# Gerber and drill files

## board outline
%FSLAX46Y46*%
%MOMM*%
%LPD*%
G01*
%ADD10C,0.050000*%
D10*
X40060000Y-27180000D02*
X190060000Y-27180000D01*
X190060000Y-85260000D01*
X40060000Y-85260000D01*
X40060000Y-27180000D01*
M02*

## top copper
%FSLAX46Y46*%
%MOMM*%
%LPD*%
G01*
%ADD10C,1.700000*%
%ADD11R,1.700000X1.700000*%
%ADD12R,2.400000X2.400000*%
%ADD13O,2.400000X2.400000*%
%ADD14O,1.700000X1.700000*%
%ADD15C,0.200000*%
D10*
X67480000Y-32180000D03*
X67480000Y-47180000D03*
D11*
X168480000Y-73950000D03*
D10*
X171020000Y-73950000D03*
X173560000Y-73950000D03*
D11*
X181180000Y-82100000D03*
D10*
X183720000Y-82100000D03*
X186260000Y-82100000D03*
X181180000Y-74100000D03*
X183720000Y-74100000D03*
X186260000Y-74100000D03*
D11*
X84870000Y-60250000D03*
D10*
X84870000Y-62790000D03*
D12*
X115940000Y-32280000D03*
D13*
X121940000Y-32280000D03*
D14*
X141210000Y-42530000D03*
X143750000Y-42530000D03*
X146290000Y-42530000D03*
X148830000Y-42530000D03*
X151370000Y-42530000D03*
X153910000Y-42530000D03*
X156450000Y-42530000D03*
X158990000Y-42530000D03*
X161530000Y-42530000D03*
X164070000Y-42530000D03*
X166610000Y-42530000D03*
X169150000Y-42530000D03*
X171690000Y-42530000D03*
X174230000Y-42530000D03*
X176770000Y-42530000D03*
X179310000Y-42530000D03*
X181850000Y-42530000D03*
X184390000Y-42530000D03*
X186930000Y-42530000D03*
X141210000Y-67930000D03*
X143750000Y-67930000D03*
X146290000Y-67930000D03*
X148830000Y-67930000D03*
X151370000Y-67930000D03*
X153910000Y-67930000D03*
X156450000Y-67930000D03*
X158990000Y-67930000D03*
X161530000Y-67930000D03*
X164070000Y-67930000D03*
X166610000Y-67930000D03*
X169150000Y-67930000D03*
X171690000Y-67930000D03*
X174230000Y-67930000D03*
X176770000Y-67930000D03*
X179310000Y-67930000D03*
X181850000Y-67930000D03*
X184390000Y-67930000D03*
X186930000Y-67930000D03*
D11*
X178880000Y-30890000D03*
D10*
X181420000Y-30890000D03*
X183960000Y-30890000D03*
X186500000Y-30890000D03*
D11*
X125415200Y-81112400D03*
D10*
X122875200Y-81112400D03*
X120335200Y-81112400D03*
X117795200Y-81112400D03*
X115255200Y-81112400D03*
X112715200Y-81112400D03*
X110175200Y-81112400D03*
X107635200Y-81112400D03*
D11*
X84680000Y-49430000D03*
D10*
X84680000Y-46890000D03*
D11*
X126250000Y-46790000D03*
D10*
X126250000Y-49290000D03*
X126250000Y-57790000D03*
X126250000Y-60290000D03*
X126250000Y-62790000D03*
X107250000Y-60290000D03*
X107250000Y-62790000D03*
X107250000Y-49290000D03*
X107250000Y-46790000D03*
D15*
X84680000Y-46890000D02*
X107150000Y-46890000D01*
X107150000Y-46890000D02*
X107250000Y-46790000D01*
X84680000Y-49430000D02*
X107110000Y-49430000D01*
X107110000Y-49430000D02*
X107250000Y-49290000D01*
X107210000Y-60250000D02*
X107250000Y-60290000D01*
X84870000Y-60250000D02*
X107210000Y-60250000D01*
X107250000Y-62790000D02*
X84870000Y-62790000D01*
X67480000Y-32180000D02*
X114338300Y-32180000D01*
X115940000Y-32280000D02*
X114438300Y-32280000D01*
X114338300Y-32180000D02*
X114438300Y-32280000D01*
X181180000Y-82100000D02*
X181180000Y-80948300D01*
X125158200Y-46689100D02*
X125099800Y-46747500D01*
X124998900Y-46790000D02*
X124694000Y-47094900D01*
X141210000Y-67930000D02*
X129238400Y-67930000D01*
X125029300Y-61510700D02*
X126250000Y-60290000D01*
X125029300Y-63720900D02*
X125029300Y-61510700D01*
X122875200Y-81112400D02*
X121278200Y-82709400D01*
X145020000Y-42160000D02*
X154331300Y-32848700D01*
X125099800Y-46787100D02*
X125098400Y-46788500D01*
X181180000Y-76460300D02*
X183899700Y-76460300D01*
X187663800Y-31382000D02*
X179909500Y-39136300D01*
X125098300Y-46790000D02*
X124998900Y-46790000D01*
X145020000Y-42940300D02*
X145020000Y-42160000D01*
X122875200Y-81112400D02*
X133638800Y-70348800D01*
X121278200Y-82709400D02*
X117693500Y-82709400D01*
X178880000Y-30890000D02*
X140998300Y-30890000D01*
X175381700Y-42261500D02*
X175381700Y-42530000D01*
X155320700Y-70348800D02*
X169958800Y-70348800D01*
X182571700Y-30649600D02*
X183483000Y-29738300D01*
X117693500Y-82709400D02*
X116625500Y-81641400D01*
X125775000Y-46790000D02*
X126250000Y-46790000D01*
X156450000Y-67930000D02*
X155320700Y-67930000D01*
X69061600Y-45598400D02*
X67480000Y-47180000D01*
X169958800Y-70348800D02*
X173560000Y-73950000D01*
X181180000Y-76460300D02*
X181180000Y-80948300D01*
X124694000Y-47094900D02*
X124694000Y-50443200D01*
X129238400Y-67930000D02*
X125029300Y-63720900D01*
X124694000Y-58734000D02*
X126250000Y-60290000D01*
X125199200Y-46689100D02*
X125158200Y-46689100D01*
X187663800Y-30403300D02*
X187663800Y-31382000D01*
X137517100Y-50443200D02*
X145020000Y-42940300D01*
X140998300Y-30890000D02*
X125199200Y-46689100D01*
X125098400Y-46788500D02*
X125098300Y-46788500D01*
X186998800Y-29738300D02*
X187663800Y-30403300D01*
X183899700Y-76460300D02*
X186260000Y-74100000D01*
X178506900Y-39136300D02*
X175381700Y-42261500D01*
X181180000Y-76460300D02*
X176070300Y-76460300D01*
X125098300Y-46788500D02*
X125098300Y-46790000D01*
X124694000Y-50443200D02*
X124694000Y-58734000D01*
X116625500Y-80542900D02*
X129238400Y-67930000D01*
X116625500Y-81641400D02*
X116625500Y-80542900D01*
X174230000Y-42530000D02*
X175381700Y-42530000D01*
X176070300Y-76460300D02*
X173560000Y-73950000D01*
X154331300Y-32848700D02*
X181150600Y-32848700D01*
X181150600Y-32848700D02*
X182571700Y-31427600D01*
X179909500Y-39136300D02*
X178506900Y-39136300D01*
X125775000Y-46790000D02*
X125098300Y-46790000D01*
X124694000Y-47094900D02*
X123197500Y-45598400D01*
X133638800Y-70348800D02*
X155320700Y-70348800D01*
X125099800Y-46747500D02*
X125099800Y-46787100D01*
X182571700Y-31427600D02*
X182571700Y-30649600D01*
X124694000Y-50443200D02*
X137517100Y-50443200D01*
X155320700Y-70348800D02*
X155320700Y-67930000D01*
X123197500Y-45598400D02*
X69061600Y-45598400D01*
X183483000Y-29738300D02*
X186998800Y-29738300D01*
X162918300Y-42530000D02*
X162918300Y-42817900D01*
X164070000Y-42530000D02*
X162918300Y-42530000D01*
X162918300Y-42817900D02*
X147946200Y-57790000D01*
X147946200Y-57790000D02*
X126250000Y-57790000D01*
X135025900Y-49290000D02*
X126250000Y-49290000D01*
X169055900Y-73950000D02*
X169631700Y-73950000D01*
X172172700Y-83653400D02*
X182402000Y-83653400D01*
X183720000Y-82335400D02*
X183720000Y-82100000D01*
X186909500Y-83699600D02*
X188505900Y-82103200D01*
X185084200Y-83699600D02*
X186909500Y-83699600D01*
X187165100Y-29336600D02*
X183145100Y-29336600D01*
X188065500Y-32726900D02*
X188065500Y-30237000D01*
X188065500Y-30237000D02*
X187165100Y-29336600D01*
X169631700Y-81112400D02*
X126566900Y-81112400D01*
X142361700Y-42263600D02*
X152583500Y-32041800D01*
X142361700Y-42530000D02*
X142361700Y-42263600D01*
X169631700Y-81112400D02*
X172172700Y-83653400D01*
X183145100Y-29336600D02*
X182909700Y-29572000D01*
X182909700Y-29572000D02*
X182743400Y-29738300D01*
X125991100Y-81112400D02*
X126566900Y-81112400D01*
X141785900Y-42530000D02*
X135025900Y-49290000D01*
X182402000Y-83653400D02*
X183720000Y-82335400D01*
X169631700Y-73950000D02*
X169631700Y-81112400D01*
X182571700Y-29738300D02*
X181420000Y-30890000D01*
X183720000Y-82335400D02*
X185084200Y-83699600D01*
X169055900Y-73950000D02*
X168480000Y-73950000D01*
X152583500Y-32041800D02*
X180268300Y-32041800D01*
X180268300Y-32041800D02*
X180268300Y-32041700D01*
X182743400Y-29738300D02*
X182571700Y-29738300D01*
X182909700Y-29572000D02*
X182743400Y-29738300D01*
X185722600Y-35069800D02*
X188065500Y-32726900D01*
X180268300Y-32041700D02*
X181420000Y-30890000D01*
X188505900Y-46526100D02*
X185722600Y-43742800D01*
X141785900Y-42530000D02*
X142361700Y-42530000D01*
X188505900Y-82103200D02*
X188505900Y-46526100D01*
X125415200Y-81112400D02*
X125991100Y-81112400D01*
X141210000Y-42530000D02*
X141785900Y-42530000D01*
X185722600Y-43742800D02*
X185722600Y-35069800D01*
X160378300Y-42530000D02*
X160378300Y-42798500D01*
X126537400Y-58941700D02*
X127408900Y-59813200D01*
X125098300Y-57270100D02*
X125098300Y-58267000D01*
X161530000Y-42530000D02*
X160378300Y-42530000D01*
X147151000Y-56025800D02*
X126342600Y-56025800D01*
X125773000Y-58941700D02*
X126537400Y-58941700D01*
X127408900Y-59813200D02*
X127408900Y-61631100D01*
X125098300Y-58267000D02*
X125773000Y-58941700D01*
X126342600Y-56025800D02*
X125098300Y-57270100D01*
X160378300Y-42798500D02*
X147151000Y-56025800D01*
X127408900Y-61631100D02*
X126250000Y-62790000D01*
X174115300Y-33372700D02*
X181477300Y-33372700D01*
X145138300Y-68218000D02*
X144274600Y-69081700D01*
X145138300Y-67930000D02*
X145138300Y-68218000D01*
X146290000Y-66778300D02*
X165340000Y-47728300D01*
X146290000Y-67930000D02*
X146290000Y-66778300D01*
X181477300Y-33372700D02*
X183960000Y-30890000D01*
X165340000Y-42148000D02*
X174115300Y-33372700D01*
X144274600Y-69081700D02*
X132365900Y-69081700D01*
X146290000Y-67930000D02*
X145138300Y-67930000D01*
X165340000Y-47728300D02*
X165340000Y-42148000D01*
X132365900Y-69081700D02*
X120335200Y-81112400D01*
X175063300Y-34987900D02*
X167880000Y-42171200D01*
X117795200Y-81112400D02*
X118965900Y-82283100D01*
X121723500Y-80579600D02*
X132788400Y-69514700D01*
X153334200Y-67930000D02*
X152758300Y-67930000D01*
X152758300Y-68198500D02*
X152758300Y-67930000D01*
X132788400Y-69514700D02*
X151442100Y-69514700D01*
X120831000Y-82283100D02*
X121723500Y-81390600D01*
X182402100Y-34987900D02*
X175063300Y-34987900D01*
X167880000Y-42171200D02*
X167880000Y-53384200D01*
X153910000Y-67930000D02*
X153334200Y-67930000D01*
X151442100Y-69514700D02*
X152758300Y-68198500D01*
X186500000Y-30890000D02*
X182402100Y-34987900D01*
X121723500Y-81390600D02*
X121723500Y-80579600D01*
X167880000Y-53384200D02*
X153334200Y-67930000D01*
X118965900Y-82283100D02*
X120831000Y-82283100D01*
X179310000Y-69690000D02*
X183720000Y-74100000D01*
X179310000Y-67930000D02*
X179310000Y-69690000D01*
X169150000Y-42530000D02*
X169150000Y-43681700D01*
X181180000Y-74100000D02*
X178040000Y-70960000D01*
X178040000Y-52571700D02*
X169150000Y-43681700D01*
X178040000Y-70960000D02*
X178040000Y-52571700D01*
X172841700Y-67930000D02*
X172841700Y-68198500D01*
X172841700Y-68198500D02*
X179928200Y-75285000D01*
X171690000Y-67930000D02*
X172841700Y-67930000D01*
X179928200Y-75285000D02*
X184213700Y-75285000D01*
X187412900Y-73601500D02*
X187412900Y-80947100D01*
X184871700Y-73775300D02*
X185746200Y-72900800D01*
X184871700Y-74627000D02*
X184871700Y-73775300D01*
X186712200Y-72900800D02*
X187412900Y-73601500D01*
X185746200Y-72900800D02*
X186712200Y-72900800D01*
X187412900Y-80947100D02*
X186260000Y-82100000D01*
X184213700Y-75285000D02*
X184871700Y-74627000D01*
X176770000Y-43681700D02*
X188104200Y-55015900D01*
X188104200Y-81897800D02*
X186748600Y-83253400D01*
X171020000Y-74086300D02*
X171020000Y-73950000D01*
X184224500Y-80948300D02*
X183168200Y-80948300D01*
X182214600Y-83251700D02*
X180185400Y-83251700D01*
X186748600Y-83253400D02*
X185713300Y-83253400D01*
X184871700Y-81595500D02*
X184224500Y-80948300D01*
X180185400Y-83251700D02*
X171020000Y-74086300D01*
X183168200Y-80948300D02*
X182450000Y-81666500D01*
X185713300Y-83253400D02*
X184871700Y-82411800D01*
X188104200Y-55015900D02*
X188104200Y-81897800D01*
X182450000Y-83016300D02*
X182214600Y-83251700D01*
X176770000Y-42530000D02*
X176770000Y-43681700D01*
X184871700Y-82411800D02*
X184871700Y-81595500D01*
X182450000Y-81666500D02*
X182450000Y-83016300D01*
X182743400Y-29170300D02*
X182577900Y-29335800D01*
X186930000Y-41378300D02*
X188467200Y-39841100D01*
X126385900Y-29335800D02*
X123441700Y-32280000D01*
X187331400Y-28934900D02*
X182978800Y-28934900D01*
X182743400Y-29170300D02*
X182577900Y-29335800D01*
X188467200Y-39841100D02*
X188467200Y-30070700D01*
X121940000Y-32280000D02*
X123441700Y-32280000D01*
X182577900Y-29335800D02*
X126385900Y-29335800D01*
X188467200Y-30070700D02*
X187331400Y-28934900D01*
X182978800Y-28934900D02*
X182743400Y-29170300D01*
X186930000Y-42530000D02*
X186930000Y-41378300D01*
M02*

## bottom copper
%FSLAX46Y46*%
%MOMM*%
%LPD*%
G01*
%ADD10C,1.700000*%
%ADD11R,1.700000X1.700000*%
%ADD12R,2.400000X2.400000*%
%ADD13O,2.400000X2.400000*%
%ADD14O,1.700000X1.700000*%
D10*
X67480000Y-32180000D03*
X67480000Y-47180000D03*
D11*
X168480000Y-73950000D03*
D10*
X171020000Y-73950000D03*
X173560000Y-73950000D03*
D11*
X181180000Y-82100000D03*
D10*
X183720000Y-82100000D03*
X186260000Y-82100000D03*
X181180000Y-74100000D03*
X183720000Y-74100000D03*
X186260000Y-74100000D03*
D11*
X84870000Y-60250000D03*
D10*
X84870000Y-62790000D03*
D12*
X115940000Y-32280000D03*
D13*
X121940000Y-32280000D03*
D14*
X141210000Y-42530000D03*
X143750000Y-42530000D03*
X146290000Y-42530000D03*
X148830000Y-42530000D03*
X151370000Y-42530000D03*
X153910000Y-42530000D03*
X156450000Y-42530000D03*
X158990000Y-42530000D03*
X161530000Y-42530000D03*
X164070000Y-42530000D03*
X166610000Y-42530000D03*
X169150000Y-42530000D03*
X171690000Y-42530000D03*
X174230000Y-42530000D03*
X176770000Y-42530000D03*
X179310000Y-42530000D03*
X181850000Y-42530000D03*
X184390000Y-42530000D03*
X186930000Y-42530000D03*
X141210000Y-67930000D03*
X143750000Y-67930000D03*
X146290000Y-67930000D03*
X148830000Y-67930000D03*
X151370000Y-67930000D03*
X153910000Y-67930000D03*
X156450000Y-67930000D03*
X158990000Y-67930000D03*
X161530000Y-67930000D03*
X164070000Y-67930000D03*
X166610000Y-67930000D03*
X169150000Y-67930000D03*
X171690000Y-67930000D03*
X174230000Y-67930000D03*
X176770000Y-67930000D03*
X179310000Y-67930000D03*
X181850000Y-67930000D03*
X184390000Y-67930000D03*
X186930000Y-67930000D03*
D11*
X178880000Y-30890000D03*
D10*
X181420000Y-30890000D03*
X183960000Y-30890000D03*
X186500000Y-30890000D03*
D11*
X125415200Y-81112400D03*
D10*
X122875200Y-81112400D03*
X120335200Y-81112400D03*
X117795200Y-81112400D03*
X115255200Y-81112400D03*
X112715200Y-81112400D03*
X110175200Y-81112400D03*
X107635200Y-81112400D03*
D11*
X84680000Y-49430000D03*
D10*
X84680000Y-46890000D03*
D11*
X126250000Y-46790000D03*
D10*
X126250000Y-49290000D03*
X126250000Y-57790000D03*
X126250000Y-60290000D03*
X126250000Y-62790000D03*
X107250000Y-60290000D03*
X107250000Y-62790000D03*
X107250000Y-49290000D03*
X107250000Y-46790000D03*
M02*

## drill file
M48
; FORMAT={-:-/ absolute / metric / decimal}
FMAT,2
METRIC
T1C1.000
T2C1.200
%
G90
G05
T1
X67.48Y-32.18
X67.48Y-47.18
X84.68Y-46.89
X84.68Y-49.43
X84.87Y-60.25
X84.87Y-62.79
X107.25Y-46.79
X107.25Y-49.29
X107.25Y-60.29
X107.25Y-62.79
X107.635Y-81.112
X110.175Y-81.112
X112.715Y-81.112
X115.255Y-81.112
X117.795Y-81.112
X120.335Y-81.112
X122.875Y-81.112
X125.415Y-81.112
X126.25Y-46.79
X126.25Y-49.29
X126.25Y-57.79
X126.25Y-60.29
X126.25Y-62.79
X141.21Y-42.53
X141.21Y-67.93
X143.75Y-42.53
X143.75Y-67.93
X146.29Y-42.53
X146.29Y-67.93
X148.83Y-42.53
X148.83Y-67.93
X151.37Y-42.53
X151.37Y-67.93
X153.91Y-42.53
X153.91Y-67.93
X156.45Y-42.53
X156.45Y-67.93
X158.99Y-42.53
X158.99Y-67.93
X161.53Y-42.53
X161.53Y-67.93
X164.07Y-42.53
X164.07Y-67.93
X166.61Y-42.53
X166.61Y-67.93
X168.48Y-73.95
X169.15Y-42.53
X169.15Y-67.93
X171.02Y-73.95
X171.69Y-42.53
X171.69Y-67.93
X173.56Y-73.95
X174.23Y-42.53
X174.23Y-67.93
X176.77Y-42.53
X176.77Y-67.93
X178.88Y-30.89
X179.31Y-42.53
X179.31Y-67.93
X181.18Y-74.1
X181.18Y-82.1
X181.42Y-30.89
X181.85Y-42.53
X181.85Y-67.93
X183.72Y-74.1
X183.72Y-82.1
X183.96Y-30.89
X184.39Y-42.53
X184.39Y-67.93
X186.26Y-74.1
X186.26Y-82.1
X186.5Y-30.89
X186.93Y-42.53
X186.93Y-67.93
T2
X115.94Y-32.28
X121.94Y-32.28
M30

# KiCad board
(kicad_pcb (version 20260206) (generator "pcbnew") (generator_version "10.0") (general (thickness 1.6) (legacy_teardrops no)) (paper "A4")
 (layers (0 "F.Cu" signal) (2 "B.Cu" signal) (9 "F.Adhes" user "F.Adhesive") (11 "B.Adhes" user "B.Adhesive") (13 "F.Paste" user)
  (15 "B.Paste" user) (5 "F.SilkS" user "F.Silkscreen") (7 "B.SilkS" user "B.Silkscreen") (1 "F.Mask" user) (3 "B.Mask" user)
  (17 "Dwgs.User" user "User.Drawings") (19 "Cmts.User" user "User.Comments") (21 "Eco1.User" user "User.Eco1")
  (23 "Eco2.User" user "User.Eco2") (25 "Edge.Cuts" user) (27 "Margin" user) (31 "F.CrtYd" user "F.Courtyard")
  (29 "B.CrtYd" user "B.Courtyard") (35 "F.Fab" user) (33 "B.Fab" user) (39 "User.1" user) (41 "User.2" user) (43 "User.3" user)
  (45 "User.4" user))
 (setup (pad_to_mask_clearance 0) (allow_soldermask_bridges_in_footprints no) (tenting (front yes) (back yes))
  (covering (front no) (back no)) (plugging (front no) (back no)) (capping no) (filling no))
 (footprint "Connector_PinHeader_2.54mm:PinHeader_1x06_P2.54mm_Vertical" (layer "F.Cu") (at 67.48 47.18 180)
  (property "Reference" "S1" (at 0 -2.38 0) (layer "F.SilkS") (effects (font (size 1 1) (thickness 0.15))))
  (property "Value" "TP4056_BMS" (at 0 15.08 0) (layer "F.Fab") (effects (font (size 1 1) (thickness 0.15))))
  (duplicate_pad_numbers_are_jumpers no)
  (pad "5" thru_hole circle (at 0 15 180) (size 1.7 1.7) (drill 1) (layers "*.Cu" "*.Mask") (remove_unused_layers no) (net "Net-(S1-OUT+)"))
  (pad "6" thru_hole circle (at 0 0 180) (size 1.7 1.7) (drill 1) (layers "*.Cu" "*.Mask") (remove_unused_layers no) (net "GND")))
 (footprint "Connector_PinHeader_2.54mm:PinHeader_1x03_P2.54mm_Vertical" (layer "F.Cu") (at 168.48 73.95 90)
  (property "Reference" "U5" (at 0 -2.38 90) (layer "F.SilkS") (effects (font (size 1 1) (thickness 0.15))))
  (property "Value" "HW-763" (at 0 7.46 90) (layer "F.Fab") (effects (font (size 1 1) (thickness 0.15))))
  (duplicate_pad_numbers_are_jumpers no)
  (pad "1" thru_hole rect (at 0 0 90) (size 1.7 1.7) (drill 1) (layers "*.Cu" "*.Mask") (remove_unused_layers no) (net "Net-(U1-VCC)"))
  (pad "2" thru_hole circle (at 0 2.54 90) (size 1.7 1.7) (drill 1) (layers "*.Cu" "*.Mask") (remove_unused_layers no) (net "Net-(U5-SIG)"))
  (pad "3" thru_hole circle (at 0 5.08 90) (size 1.7 1.7) (drill 1) (layers "*.Cu" "*.Mask") (remove_unused_layers no) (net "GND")))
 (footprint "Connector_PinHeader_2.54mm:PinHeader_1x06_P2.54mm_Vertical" (layer "F.Cu") (at 181.18 82.1 90)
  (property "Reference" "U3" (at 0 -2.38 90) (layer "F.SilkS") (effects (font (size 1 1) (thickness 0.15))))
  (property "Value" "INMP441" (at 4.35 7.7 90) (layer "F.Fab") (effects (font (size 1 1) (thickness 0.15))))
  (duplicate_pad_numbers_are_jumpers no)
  (pad "1" thru_hole rect (at 0 0 90) (size 1.7 1.7) (drill 1) (layers "*.Cu" "*.Mask") (remove_unused_layers no) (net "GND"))
  (pad "2" thru_hole circle (at 0 2.54 90) (size 1.7 1.7) (drill 1) (layers "*.Cu" "*.Mask") (remove_unused_layers no) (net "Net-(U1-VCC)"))
  (pad "3" thru_hole circle (at 0 5.08 90) (size 1.7 1.7) (drill 1) (layers "*.Cu" "*.Mask") (remove_unused_layers no) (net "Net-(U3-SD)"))
  (pad "4" thru_hole circle (at 8 0 90) (size 1.7 1.7) (drill 1) (layers "*.Cu" "*.Mask") (remove_unused_layers no) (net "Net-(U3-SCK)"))
  (pad "5" thru_hole circle (at 8 2.54 90) (size 1.7 1.7) (drill 1) (layers "*.Cu" "*.Mask") (remove_unused_layers no) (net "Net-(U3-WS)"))
  (pad "6" thru_hole circle (at 8 5.08 90) (size 1.7 1.7) (drill 1) (layers "*.Cu" "*.Mask") (remove_unused_layers no) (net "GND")))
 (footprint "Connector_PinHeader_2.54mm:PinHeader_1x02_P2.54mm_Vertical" (layer "F.Cu") (at 84.87 60.25)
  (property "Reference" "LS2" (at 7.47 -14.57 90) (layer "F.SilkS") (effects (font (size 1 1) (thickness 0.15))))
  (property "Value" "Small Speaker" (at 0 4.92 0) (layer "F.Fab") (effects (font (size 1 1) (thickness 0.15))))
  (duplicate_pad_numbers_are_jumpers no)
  (pad "1" thru_hole rect (at 0 0) (size 1.7 1.7) (drill 1) (layers "*.Cu" "*.Mask") (remove_unused_layers no) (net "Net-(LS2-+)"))
  (pad "2" thru_hole circle (at 0 2.54) (size 1.7 1.7) (drill 1) (layers "*.Cu" "*.Mask") (remove_unused_layers no) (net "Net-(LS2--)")))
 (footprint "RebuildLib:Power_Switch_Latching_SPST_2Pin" (layer "F.Cu") (at 115.94 32.28)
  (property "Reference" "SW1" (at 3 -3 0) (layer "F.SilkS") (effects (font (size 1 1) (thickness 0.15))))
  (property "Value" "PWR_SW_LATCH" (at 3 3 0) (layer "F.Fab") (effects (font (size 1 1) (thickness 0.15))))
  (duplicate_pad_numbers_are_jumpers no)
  (pad "1" thru_hole rect (at 0 0) (size 2.4 2.4) (drill 1.2) (layers "*.Cu" "*.Mask") (remove_unused_layers no) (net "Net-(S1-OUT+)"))
  (pad "2" thru_hole oval (at 6 0) (size 2.4 2.4) (drill 1.2) (layers "*.Cu" "*.Mask") (remove_unused_layers no) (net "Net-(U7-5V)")))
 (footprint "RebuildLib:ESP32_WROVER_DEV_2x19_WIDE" (layer "F.Cu") (at 164.07 55.23 -90)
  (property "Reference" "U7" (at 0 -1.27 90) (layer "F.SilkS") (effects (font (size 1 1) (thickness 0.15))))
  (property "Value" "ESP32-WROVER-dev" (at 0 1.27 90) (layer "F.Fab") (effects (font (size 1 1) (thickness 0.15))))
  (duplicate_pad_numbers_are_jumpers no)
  (pad "1" thru_hole oval (at -12.7 22.86 270) (size 1.7 1.7) (drill 1) (layers "*.Cu" "*.Mask") (remove_unused_layers no)
   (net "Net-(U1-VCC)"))
  (pad "2" thru_hole oval (at -12.7 20.32 270) (size 1.7 1.7) (drill 1) (layers "*.Cu" "*.Mask") (remove_unused_layers no)
   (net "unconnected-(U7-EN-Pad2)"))
  (pad "3" thru_hole oval (at -12.7 17.78 270) (size 1.7 1.7) (drill 1) (layers "*.Cu" "*.Mask") (remove_unused_layers no)
   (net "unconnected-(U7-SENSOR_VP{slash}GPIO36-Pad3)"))
  (pad "4" thru_hole oval (at -12.7 15.24 270) (size 1.7 1.7) (drill 1) (layers "*.Cu" "*.Mask") (remove_unused_layers no)
   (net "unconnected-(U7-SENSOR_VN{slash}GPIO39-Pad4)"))
  (pad "5" thru_hole oval (at -12.7 12.7 270) (size 1.7 1.7) (drill 1) (layers "*.Cu" "*.Mask") (remove_unused_layers no)
   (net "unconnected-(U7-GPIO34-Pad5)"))
  (pad "6" thru_hole oval (at -12.7 10.16 270) (size 1.7 1.7) (drill 1) (layers "*.Cu" "*.Mask") (remove_unused_layers no)
   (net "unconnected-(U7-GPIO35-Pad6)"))
  (pad "7" thru_hole oval (at -12.7 7.62 270) (size 1.7 1.7) (drill 1) (layers "*.Cu" "*.Mask") (remove_unused_layers no)
   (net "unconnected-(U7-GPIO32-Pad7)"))
  (pad "8" thru_hole oval (at -12.7 5.08 270) (size 1.7 1.7) (drill 1) (layers "*.Cu" "*.Mask") (remove_unused_layers no)
   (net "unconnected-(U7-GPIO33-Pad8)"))
  (pad "9" thru_hole oval (at -12.7 2.54 270) (size 1.7 1.7) (drill 1) (layers "*.Cu" "*.Mask") (remove_unused_layers no)
   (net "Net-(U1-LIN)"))
  (pad "10" thru_hole oval (at -12.7 0 270) (size 1.7 1.7) (drill 1) (layers "*.Cu" "*.Mask") (remove_unused_layers no) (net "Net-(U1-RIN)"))
  (pad "11" thru_hole oval (at -12.7 -2.54 270) (size 1.7 1.7) (drill 1) (layers "*.Cu" "*.Mask") (remove_unused_layers no)
   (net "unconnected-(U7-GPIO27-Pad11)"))
  (pad "12" thru_hole oval (at -12.7 -5.08 270) (size 1.7 1.7) (drill 1) (layers "*.Cu" "*.Mask") (remove_unused_layers no)
   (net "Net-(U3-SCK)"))
  (pad "13" thru_hole oval (at -12.7 -7.62 270) (size 1.7 1.7) (drill 1) (layers "*.Cu" "*.Mask") (remove_unused_layers no)
   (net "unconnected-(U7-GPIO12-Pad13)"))
  (pad "14" thru_hole oval (at -12.7 -10.16 270) (size 1.7 1.7) (drill 1) (layers "*.Cu" "*.Mask") (remove_unused_layers no) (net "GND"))
  (pad "15" thru_hole oval (at -12.7 -12.7 270) (size 1.7 1.7) (drill 1) (layers "*.Cu" "*.Mask") (remove_unused_layers no)
   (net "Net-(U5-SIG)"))
  (pad "16" thru_hole oval (at -12.7 -15.24 270) (size 1.7 1.7) (drill 1) (layers "*.Cu" "*.Mask") (remove_unused_layers no)
   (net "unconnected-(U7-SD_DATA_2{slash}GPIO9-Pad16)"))
  (pad "17" thru_hole oval (at -12.7 -17.78 270) (size 1.7 1.7) (drill 1) (layers "*.Cu" "*.Mask") (remove_unused_layers no)
   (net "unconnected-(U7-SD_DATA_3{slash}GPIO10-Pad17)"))
  (pad "18" thru_hole oval (at -12.7 -20.32 270) (size 1.7 1.7) (drill 1) (layers "*.Cu" "*.Mask") (remove_unused_layers no)
   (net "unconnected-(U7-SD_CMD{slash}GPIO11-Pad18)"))
  (pad "19" thru_hole oval (at -12.7 -22.86 270) (size 1.7 1.7) (drill 1) (layers "*.Cu" "*.Mask") (remove_unused_layers no)
   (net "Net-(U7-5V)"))
  (pad "20" thru_hole oval (at 12.7 22.86 270) (size 1.7 1.7) (drill 1) (layers "*.Cu" "*.Mask") (remove_unused_layers no) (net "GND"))
  (pad "21" thru_hole oval (at 12.7 20.32 270) (size 1.7 1.7) (drill 1) (layers "*.Cu" "*.Mask") (remove_unused_layers no)
   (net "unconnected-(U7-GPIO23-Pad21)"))
  (pad "22" thru_hole oval (at 12.7 17.78 270) (size 1.7 1.7) (drill 1) (layers "*.Cu" "*.Mask") (remove_unused_layers no)
   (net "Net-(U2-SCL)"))
  (pad "23" thru_hole oval (at 12.7 15.24 270) (size 1.7 1.7) (drill 1) (layers "*.Cu" "*.Mask") (remove_unused_layers no)
   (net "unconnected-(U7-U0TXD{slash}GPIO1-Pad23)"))
  (pad "24" thru_hole oval (at 12.7 12.7 270) (size 1.7 1.7) (drill 1) (layers "*.Cu" "*.Mask") (remove_unused_layers no)
   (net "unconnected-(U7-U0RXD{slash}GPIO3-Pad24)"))
  (pad "25" thru_hole oval (at 12.7 10.16 270) (size 1.7 1.7) (drill 1) (layers "*.Cu" "*.Mask") (remove_unused_layers no)
   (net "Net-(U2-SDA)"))
  (pad "26" thru_hole oval (at 12.7 7.62 270) (size 1.7 1.7) (drill 1) (layers "*.Cu" "*.Mask") (remove_unused_layers no) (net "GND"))
  (pad "27" thru_hole oval (at 12.7 5.08 270) (size 1.7 1.7) (drill 1) (layers "*.Cu" "*.Mask") (remove_unused_layers no)
   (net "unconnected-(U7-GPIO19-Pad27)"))
  (pad "28" thru_hole oval (at 12.7 2.54 270) (size 1.7 1.7) (drill 1) (layers "*.Cu" "*.Mask") (remove_unused_layers no)
   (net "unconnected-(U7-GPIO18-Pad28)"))
  (pad "29" thru_hole oval (at 12.7 0 270) (size 1.7 1.7) (drill 1) (layers "*.Cu" "*.Mask") (remove_unused_layers no)
   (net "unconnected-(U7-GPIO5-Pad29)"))
  (pad "30" thru_hole oval (at 12.7 -2.54 270) (size 1.7 1.7) (drill 1) (layers "*.Cu" "*.Mask") (remove_unused_layers no)
   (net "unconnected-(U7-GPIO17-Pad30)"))
  (pad "31" thru_hole oval (at 12.7 -5.08 270) (size 1.7 1.7) (drill 1) (layers "*.Cu" "*.Mask") (remove_unused_layers no)
   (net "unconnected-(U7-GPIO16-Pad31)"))
  (pad "32" thru_hole oval (at 12.7 -7.62 270) (size 1.7 1.7) (drill 1) (layers "*.Cu" "*.Mask") (remove_unused_layers no)
   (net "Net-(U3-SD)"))
  (pad "33" thru_hole oval (at 12.7 -10.16 270) (size 1.7 1.7) (drill 1) (layers "*.Cu" "*.Mask") (remove_unused_layers no)
   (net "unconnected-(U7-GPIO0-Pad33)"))
  (pad "34" thru_hole oval (at 12.7 -12.7 270) (size 1.7 1.7) (drill 1) (layers "*.Cu" "*.Mask") (remove_unused_layers no)
   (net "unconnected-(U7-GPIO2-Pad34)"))
  (pad "35" thru_hole oval (at 12.7 -15.24 270) (size 1.7 1.7) (drill 1) (layers "*.Cu" "*.Mask") (remove_unused_layers no)
   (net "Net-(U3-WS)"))
  (pad "36" thru_hole oval (at 12.7 -17.78 270) (size 1.7 1.7) (drill 1) (layers "*.Cu" "*.Mask") (remove_unused_layers no)
   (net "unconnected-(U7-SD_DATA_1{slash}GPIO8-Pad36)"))
  (pad "37" thru_hole oval (at 12.7 -20.32 270) (size 1.7 1.7) (drill 1) (layers "*.Cu" "*.Mask") (remove_unused_layers no)
   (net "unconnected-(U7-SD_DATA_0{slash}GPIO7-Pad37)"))
  (pad "38" thru_hole oval (at 12.7 -22.86 270) (size 1.7 1.7) (drill 1) (layers "*.Cu" "*.Mask") (remove_unused_layers no)
   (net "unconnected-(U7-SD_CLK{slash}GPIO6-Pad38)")))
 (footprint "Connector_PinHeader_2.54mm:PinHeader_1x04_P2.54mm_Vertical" (layer "F.Cu") (at 178.88 30.89 90)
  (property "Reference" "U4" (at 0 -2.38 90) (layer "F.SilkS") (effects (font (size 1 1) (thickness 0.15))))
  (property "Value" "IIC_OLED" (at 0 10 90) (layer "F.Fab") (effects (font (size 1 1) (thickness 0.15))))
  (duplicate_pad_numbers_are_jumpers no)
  (pad "1" thru_hole rect (at 0 0 90) (size 1.7 1.7) (drill 1) (layers "*.Cu" "*.Mask") (remove_unused_layers no) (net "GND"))
  (pad "2" thru_hole circle (at 0 2.54 90) (size 1.7 1.7) (drill 1) (layers "*.Cu" "*.Mask") (remove_unused_layers no) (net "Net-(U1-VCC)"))
  (pad "3" thru_hole circle (at 0 5.08 90) (size 1.7 1.7) (drill 1) (layers "*.Cu" "*.Mask") (remove_unused_layers no) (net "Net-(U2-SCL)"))
  (pad "4" thru_hole circle (at 0 7.62 90) (size 1.7 1.7) (drill 1) (layers "*.Cu" "*.Mask") (remove_unused_layers no) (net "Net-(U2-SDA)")))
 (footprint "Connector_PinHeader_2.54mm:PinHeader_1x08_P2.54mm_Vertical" (layer "F.Cu") (at 125.4152 81.1124 -90)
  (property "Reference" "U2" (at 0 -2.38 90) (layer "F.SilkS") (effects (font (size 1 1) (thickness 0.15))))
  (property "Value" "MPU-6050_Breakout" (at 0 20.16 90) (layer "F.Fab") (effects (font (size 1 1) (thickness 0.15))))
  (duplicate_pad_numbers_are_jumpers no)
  (pad "1" thru_hole rect (at 0 0 270) (size 1.7 1.7) (drill 1) (layers "*.Cu" "*.Mask") (remove_unused_layers no) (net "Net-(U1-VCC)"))
  (pad "2" thru_hole circle (at 0 2.54 270) (size 1.7 1.7) (drill 1) (layers "*.Cu" "*.Mask") (remove_unused_layers no) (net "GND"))
  (pad "3" thru_hole circle (at 0 5.08 270) (size 1.7 1.7) (drill 1) (layers "*.Cu" "*.Mask") (remove_unused_layers no) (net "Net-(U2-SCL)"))
  (pad "4" thru_hole circle (at 0 7.62 270) (size 1.7 1.7) (drill 1) (layers "*.Cu" "*.Mask") (remove_unused_layers no) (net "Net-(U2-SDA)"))
  (pad "5" thru_hole circle (at 0 10.16 270) (size 1.7 1.7) (drill 1) (layers "*.Cu" "*.Mask") (remove_unused_layers no)
   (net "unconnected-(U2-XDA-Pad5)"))
  (pad "6" thru_hole circle (at 0 12.7 270) (size 1.7 1.7) (drill 1) (layers "*.Cu" "*.Mask") (remove_unused_layers no)
   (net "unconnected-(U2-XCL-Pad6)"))
  (pad "7" thru_hole circle (at 0 15.24 270) (size 1.7 1.7) (drill 1) (layers "*.Cu" "*.Mask") (remove_unused_layers no)
   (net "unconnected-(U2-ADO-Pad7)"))
  (pad "8" thru_hole circle (at 0 17.78 270) (size 1.7 1.7) (drill 1) (layers "*.Cu" "*.Mask") (remove_unused_layers no)
   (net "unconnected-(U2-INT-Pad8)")))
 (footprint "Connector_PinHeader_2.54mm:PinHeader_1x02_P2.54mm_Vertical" (layer "F.Cu") (at 84.68 49.43 180)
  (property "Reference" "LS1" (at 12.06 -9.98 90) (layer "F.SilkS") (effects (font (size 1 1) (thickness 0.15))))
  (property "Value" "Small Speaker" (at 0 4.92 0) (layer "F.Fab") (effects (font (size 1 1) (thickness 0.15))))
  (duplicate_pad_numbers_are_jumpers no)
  (pad "1" thru_hole rect (at 0 0 180) (size 1.7 1.7) (drill 1) (layers "*.Cu" "*.Mask") (remove_unused_layers no) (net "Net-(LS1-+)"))
  (pad "2" thru_hole circle (at 0 2.54 180) (size 1.7 1.7) (drill 1) (layers "*.Cu" "*.Mask") (remove_unused_layers no) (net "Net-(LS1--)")))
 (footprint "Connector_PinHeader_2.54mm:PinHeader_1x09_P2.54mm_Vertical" (layer "F.Cu") (at 126.25 46.79 -90)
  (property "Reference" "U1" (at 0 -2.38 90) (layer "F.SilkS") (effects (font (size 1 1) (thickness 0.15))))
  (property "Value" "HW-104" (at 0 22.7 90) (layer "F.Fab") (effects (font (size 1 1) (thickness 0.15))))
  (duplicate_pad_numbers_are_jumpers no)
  (pad "1" thru_hole rect (at 0 0 270) (size 1.7 1.7) (drill 1) (layers "*.Cu" "*.Mask") (remove_unused_layers no) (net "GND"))
  (pad "2" thru_hole circle (at 2.5 0 270) (size 1.7 1.7) (drill 1) (layers "*.Cu" "*.Mask") (remove_unused_layers no) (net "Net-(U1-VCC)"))
  (pad "3" thru_hole circle (at 11 0 270) (size 1.7 1.7) (drill 1) (layers "*.Cu" "*.Mask") (remove_unused_layers no) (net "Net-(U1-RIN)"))
  (pad "4" thru_hole circle (at 13.5 0 270) (size 1.7 1.7) (drill 1) (layers "*.Cu" "*.Mask") (remove_unused_layers no) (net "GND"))
  (pad "5" thru_hole circle (at 16 0 270) (size 1.7 1.7) (drill 1) (layers "*.Cu" "*.Mask") (remove_unused_layers no) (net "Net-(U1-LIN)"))
  (pad "6" thru_hole circle (at 13.5 19 270) (size 1.7 1.7) (drill 1) (layers "*.Cu" "*.Mask") (remove_unused_layers no) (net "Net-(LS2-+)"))
  (pad "7" thru_hole circle (at 16 19 270) (size 1.7 1.7) (drill 1) (layers "*.Cu" "*.Mask") (remove_unused_layers no) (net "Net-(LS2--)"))
  (pad "8" thru_hole circle (at 2.5 19 270) (size 1.7 1.7) (drill 1) (layers "*.Cu" "*.Mask") (remove_unused_layers no) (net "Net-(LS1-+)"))
  (pad "9" thru_hole circle (at 0 19 270) (size 1.7 1.7) (drill 1) (layers "*.Cu" "*.Mask") (remove_unused_layers no) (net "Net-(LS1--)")))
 (gr_rect (start 40.06 27.18) (end 190.06 85.26) (stroke (width 0.05) (type default)) (fill no) (layer "Edge.Cuts"))
 (segment (start 84.68 46.89) (end 107.15 46.89) (width 0.2) (layer "F.Cu") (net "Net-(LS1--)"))
 (segment (start 107.15 46.89) (end 107.25 46.79) (width 0.2) (layer "F.Cu") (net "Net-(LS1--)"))
 (segment (start 84.68 49.43) (end 107.11 49.43) (width 0.2) (layer "F.Cu") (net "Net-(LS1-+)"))
 (segment (start 107.11 49.43) (end 107.25 49.29) (width 0.2) (layer "F.Cu") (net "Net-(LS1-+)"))
 (segment (start 107.21 60.25) (end 107.25 60.29) (width 0.2) (layer "F.Cu") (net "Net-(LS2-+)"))
 (segment (start 84.87 60.25) (end 107.21 60.25) (width 0.2) (layer "F.Cu") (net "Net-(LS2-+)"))
 (segment (start 107.25 62.79) (end 84.87 62.79) (width 0.2) (layer "F.Cu") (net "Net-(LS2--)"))
 (segment (start 67.48 32.18) (end 114.3383 32.18) (width 0.2) (layer "F.Cu") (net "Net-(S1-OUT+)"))
 (segment (start 115.94 32.28) (end 114.4383 32.28) (width 0.2) (layer "F.Cu") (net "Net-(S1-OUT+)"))
 (segment (start 114.3383 32.18) (end 114.4383 32.28) (width 0.2) (layer "F.Cu") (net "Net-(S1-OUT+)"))
 (segment (start 181.18 82.1) (end 181.18 80.9483) (width 0.2) (layer "F.Cu") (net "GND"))
 (segment (start 125.1582 46.6891) (end 125.0998 46.7475) (width 0.2) (layer "F.Cu") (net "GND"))
 (segment (start 124.9989 46.79) (end 124.694 47.0949) (width 0.2) (layer "F.Cu") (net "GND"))
 (segment (start 141.21 67.93) (end 129.2384 67.93) (width 0.2) (layer "F.Cu") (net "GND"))
 (segment (start 125.0293 61.5107) (end 126.25 60.29) (width 0.2) (layer "F.Cu") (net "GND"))
 (segment (start 125.0293 63.7209) (end 125.0293 61.5107) (width 0.2) (layer "F.Cu") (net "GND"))
 (segment (start 122.8752 81.1124) (end 121.2782 82.7094) (width 0.2) (layer "F.Cu") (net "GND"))
 (segment (start 145.02 42.16) (end 154.3313 32.8487) (width 0.2) (layer "F.Cu") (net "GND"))
 (segment (start 125.0998 46.7871) (end 125.0984 46.7885) (width 0.2) (layer "F.Cu") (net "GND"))
 (segment (start 181.18 76.4603) (end 183.8997 76.4603) (width 0.2) (layer "F.Cu") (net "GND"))
 (segment (start 187.6638 31.382) (end 179.9095 39.1363) (width 0.2) (layer "F.Cu") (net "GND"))
 (segment (start 125.0983 46.79) (end 124.9989 46.79) (width 0.2) (layer "F.Cu") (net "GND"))
 (segment (start 145.02 42.9403) (end 145.02 42.16) (width 0.2) (layer "F.Cu") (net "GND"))
 (segment (start 122.8752 81.1124) (end 133.6388 70.3488) (width 0.2) (layer "F.Cu") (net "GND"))
 (segment (start 121.2782 82.7094) (end 117.6935 82.7094) (width 0.2) (layer "F.Cu") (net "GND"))
 (segment (start 178.88 30.89) (end 140.9983 30.89) (width 0.2) (layer "F.Cu") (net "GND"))
 (segment (start 175.3817 42.2615) (end 175.3817 42.53) (width 0.2) (layer "F.Cu") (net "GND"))
 (segment (start 155.3207 70.3488) (end 169.9588 70.3488) (width 0.2) (layer "F.Cu") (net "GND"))
 (segment (start 182.5717 30.6496) (end 183.483 29.7383) (width 0.2) (layer "F.Cu") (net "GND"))
 (segment (start 117.6935 82.7094) (end 116.6255 81.6414) (width 0.2) (layer "F.Cu") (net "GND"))
 (segment (start 125.775 46.79) (end 126.25 46.79) (width 0.2) (layer "F.Cu") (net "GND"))
 (segment (start 156.45 67.93) (end 155.3207 67.93) (width 0.2) (layer "F.Cu") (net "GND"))
 (segment (start 69.0616 45.5984) (end 67.48 47.18) (width 0.2) (layer "F.Cu") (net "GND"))
 (segment (start 169.9588 70.3488) (end 173.56 73.95) (width 0.2) (layer "F.Cu") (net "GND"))
 (segment (start 181.18 76.4603) (end 181.18 80.9483) (width 0.2) (layer "F.Cu") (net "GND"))
 (segment (start 124.694 47.0949) (end 124.694 50.4432) (width 0.2) (layer "F.Cu") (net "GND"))
 (segment (start 129.2384 67.93) (end 125.0293 63.7209) (width 0.2) (layer "F.Cu") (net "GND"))
 (segment (start 124.694 58.734) (end 126.25 60.29) (width 0.2) (layer "F.Cu") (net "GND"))
 (segment (start 125.1992 46.6891) (end 125.1582 46.6891) (width 0.2) (layer "F.Cu") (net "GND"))
 (segment (start 187.6638 30.4033) (end 187.6638 31.382) (width 0.2) (layer "F.Cu") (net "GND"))
 (segment (start 137.5171 50.4432) (end 145.02 42.9403) (width 0.2) (layer "F.Cu") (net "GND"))
 (segment (start 140.9983 30.89) (end 125.1992 46.6891) (width 0.2) (layer "F.Cu") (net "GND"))
 (segment (start 125.0984 46.7885) (end 125.0983 46.7885) (width 0.2) (layer "F.Cu") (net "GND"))
 (segment (start 186.9988 29.7383) (end 187.6638 30.4033) (width 0.2) (layer "F.Cu") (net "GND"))
 (segment (start 183.8997 76.4603) (end 186.26 74.1) (width 0.2) (layer "F.Cu") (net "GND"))
 (segment (start 178.5069 39.1363) (end 175.3817 42.2615) (width 0.2) (layer "F.Cu") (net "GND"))
 (segment (start 181.18 76.4603) (end 176.0703 76.4603) (width 0.2) (layer "F.Cu") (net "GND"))
 (segment (start 125.0983 46.7885) (end 125.0983 46.79) (width 0.2) (layer "F.Cu") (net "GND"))
 (segment (start 124.694 50.4432) (end 124.694 58.734) (width 0.2) (layer "F.Cu") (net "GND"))
 (segment (start 116.6255 80.5429) (end 129.2384 67.93) (width 0.2) (layer "F.Cu") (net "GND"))
 (segment (start 116.6255 81.6414) (end 116.6255 80.5429) (width 0.2) (layer "F.Cu") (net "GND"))
 (segment (start 174.23 42.53) (end 175.3817 42.53) (width 0.2) (layer "F.Cu") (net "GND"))
 (segment (start 176.0703 76.4603) (end 173.56 73.95) (width 0.2) (layer "F.Cu") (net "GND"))
 (segment (start 154.3313 32.8487) (end 181.1506 32.8487) (width 0.2) (layer "F.Cu") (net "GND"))
 (segment (start 181.1506 32.8487) (end 182.5717 31.4276) (width 0.2) (layer "F.Cu") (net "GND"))
 (segment (start 179.9095 39.1363) (end 178.5069 39.1363) (width 0.2) (layer "F.Cu") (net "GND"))
 (segment (start 125.775 46.79) (end 125.0983 46.79) (width 0.2) (layer "F.Cu") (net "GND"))
 (segment (start 124.694 47.0949) (end 123.1975 45.5984) (width 0.2) (layer "F.Cu") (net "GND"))
 (segment (start 133.6388 70.3488) (end 155.3207 70.3488) (width 0.2) (layer "F.Cu") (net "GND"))
 (segment (start 125.0998 46.7475) (end 125.0998 46.7871) (width 0.2) (layer "F.Cu") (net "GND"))
 (segment (start 182.5717 31.4276) (end 182.5717 30.6496) (width 0.2) (layer "F.Cu") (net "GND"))
 (segment (start 124.694 50.4432) (end 137.5171 50.4432) (width 0.2) (layer "F.Cu") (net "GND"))
 (segment (start 155.3207 70.3488) (end 155.3207 67.93) (width 0.2) (layer "F.Cu") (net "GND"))
 (segment (start 123.1975 45.5984) (end 69.0616 45.5984) (width 0.2) (layer "F.Cu") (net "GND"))
 (segment (start 183.483 29.7383) (end 186.9988 29.7383) (width 0.2) (layer "F.Cu") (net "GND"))
 (segment (start 162.9183 42.53) (end 162.9183 42.8179) (width 0.2) (layer "F.Cu") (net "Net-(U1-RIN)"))
 (segment (start 164.07 42.53) (end 162.9183 42.53) (width 0.2) (layer "F.Cu") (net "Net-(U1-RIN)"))
 (segment (start 162.9183 42.8179) (end 147.9462 57.79) (width 0.2) (layer "F.Cu") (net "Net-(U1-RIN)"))
 (segment (start 147.9462 57.79) (end 126.25 57.79) (width 0.2) (layer "F.Cu") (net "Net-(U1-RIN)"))
 (segment (start 135.0259 49.29) (end 126.25 49.29) (width 0.2) (layer "F.Cu") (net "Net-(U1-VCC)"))
 (segment (start 169.0559 73.95) (end 169.6317 73.95) (width 0.2) (layer "F.Cu") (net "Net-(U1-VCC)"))
 (segment (start 172.1727 83.6534) (end 182.402 83.6534) (width 0.2) (layer "F.Cu") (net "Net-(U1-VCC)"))
 (segment (start 183.72 82.3354) (end 183.72 82.1) (width 0.2) (layer "F.Cu") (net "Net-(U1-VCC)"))
 (segment (start 186.9095 83.6996) (end 188.5059 82.1032) (width 0.2) (layer "F.Cu") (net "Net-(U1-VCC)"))
 (segment (start 185.0842 83.6996) (end 186.9095 83.6996) (width 0.2) (layer "F.Cu") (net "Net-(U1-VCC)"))
 (segment (start 187.1651 29.3366) (end 183.1451 29.3366) (width 0.2) (layer "F.Cu") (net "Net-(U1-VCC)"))
 (segment (start 188.0655 32.7269) (end 188.0655 30.237) (width 0.2) (layer "F.Cu") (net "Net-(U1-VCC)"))
 (segment (start 188.0655 30.237) (end 187.1651 29.3366) (width 0.2) (layer "F.Cu") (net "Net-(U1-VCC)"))
 (segment (start 169.6317 81.1124) (end 126.5669 81.1124) (width 0.2) (layer "F.Cu") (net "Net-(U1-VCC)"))
 (segment (start 142.3617 42.2636) (end 152.5835 32.0418) (width 0.2) (layer "F.Cu") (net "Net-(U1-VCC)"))
 (segment (start 142.3617 42.53) (end 142.3617 42.2636) (width 0.2) (layer "F.Cu") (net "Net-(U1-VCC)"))
 (segment (start 169.6317 81.1124) (end 172.1727 83.6534) (width 0.2) (layer "F.Cu") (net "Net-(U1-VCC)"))
 (segment (start 183.1451 29.3366) (end 182.9097 29.572) (width 0.2) (layer "F.Cu") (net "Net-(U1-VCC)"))
 (segment (start 182.9097 29.572) (end 182.7434 29.7383) (width 0.2) (layer "F.Cu") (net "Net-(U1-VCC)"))
 (segment (start 125.9911 81.1124) (end 126.5669 81.1124) (width 0.2) (layer "F.Cu") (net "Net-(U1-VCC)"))
 (segment (start 141.7859 42.53) (end 135.0259 49.29) (width 0.2) (layer "F.Cu") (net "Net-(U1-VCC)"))
 (segment (start 182.402 83.6534) (end 183.72 82.3354) (width 0.2) (layer "F.Cu") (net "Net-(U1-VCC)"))
 (segment (start 169.6317 73.95) (end 169.6317 81.1124) (width 0.2) (layer "F.Cu") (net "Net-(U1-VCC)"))
 (segment (start 182.5717 29.7383) (end 181.42 30.89) (width 0.2) (layer "F.Cu") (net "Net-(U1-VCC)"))
 (segment (start 183.72 82.3354) (end 185.0842 83.6996) (width 0.2) (layer "F.Cu") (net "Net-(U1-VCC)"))
 (segment (start 169.0559 73.95) (end 168.48 73.95) (width 0.2) (layer "F.Cu") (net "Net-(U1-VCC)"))
 (segment (start 152.5835 32.0418) (end 180.2683 32.0418) (width 0.2) (layer "F.Cu") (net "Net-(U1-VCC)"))
 (segment (start 180.2683 32.0418) (end 180.2683 32.0417) (width 0.2) (layer "F.Cu") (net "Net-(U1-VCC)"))
 (segment (start 182.7434 29.7383) (end 182.5717 29.7383) (width 0.2) (layer "F.Cu") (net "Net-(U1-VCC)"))
 (segment (start 182.9097 29.572) (end 182.7434 29.7383) (width 0.2) (layer "F.Cu") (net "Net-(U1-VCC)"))
 (segment (start 185.7226 35.0698) (end 188.0655 32.7269) (width 0.2) (layer "F.Cu") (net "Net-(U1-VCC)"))
 (segment (start 180.2683 32.0417) (end 181.42 30.89) (width 0.2) (layer "F.Cu") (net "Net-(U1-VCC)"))
 (segment (start 188.5059 46.5261) (end 185.7226 43.7428) (width 0.2) (layer "F.Cu") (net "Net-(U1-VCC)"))
 (segment (start 141.7859 42.53) (end 142.3617 42.53) (width 0.2) (layer "F.Cu") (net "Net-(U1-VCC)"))
 (segment (start 188.5059 82.1032) (end 188.5059 46.5261) (width 0.2) (layer "F.Cu") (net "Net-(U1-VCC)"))
 (segment (start 125.4152 81.1124) (end 125.9911 81.1124) (width 0.2) (layer "F.Cu") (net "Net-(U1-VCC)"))
 (segment (start 141.21 42.53) (end 141.7859 42.53) (width 0.2) (layer "F.Cu") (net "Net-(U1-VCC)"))
 (segment (start 185.7226 43.7428) (end 185.7226 35.0698) (width 0.2) (layer "F.Cu") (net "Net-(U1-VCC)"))
 (segment (start 160.3783 42.53) (end 160.3783 42.7985) (width 0.2) (layer "F.Cu") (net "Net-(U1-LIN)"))
 (segment (start 126.5374 58.9417) (end 127.4089 59.8132) (width 0.2) (layer "F.Cu") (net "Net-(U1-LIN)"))
 (segment (start 125.0983 57.2701) (end 125.0983 58.267) (width 0.2) (layer "F.Cu") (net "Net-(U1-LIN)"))
 (segment (start 161.53 42.53) (end 160.3783 42.53) (width 0.2) (layer "F.Cu") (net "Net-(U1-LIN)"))
 (segment (start 147.151 56.0258) (end 126.3426 56.0258) (width 0.2) (layer "F.Cu") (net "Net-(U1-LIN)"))
 (segment (start 125.773 58.9417) (end 126.5374 58.9417) (width 0.2) (layer "F.Cu") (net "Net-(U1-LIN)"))
 (segment (start 127.4089 59.8132) (end 127.4089 61.6311) (width 0.2) (layer "F.Cu") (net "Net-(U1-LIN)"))
 (segment (start 125.0983 58.267) (end 125.773 58.9417) (width 0.2) (layer "F.Cu") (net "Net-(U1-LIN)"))
 (segment (start 126.3426 56.0258) (end 125.0983 57.2701) (width 0.2) (layer "F.Cu") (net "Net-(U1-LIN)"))
 (segment (start 160.3783 42.7985) (end 147.151 56.0258) (width 0.2) (layer "F.Cu") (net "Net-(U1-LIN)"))
 (segment (start 127.4089 61.6311) (end 126.25 62.79) (width 0.2) (layer "F.Cu") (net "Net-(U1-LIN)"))
 (segment (start 174.1153 33.3727) (end 181.4773 33.3727) (width 0.2) (layer "F.Cu") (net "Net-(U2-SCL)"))
 (segment (start 145.1383 68.218) (end 144.2746 69.0817) (width 0.2) (layer "F.Cu") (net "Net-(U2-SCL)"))
 (segment (start 145.1383 67.93) (end 145.1383 68.218) (width 0.2) (layer "F.Cu") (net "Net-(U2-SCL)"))
 (segment (start 146.29 66.7783) (end 165.34 47.7283) (width 0.2) (layer "F.Cu") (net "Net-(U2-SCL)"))
 (segment (start 146.29 67.93) (end 146.29 66.7783) (width 0.2) (layer "F.Cu") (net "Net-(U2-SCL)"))
 (segment (start 181.4773 33.3727) (end 183.96 30.89) (width 0.2) (layer "F.Cu") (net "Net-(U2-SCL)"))
 (segment (start 165.34 42.148) (end 174.1153 33.3727) (width 0.2) (layer "F.Cu") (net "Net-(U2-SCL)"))
 (segment (start 144.2746 69.0817) (end 132.3659 69.0817) (width 0.2) (layer "F.Cu") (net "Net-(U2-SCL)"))
 (segment (start 146.29 67.93) (end 145.1383 67.93) (width 0.2) (layer "F.Cu") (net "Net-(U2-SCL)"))
 (segment (start 165.34 47.7283) (end 165.34 42.148) (width 0.2) (layer "F.Cu") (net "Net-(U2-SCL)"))
 (segment (start 132.3659 69.0817) (end 120.3352 81.1124) (width 0.2) (layer "F.Cu") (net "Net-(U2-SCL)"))
 (segment (start 175.0633 34.9879) (end 167.88 42.1712) (width 0.2) (layer "F.Cu") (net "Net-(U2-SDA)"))
 (segment (start 117.7952 81.1124) (end 118.9659 82.2831) (width 0.2) (layer "F.Cu") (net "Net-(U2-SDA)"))
 (segment (start 121.7235 80.5796) (end 132.7884 69.5147) (width 0.2) (layer "F.Cu") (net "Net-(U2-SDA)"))
 (segment (start 153.3342 67.93) (end 152.7583 67.93) (width 0.2) (layer "F.Cu") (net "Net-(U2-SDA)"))
 (segment (start 152.7583 68.1985) (end 152.7583 67.93) (width 0.2) (layer "F.Cu") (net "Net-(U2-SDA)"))
 (segment (start 132.7884 69.5147) (end 151.4421 69.5147) (width 0.2) (layer "F.Cu") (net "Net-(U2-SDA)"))
 (segment (start 120.831 82.2831) (end 121.7235 81.3906) (width 0.2) (layer "F.Cu") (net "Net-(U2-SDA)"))
 (segment (start 182.4021 34.9879) (end 175.0633 34.9879) (width 0.2) (layer "F.Cu") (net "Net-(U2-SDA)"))
 (segment (start 167.88 42.1712) (end 167.88 53.3842) (width 0.2) (layer "F.Cu") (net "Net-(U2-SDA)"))
 (segment (start 153.91 67.93) (end 153.3342 67.93) (width 0.2) (layer "F.Cu") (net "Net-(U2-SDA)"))
 (segment (start 151.4421 69.5147) (end 152.7583 68.1985) (width 0.2) (layer "F.Cu") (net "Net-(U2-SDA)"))
 (segment (start 186.5 30.89) (end 182.4021 34.9879) (width 0.2) (layer "F.Cu") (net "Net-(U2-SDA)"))
 (segment (start 121.7235 81.3906) (end 121.7235 80.5796) (width 0.2) (layer "F.Cu") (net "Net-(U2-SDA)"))
 (segment (start 167.88 53.3842) (end 153.3342 67.93) (width 0.2) (layer "F.Cu") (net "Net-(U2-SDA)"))
 (segment (start 118.9659 82.2831) (end 120.831 82.2831) (width 0.2) (layer "F.Cu") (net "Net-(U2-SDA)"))
 (segment (start 179.31 69.69) (end 183.72 74.1) (width 0.2) (layer "F.Cu") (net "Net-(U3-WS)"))
 (segment (start 179.31 67.93) (end 179.31 69.69) (width 0.2) (layer "F.Cu") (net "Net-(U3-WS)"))
 (segment (start 169.15 42.53) (end 169.15 43.6817) (width 0.2) (layer "F.Cu") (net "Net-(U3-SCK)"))
 (segment (start 181.18 74.1) (end 178.04 70.96) (width 0.2) (layer "F.Cu") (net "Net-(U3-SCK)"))
 (segment (start 178.04 52.5717) (end 169.15 43.6817) (width 0.2) (layer "F.Cu") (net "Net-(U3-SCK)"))
 (segment (start 178.04 70.96) (end 178.04 52.5717) (width 0.2) (layer "F.Cu") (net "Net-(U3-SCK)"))
 (segment (start 172.8417 67.93) (end 172.8417 68.1985) (width 0.2) (layer "F.Cu") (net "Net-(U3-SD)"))
 (segment (start 172.8417 68.1985) (end 179.9282 75.285) (width 0.2) (layer "F.Cu") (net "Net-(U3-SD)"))
 (segment (start 171.69 67.93) (end 172.8417 67.93) (width 0.2) (layer "F.Cu") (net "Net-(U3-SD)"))
 (segment (start 179.9282 75.285) (end 184.2137 75.285) (width 0.2) (layer "F.Cu") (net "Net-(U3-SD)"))
 (segment (start 187.4129 73.6015) (end 187.4129 80.9471) (width 0.2) (layer "F.Cu") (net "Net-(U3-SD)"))
 (segment (start 184.8717 73.7753) (end 185.7462 72.9008) (width 0.2) (layer "F.Cu") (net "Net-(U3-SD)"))
 (segment (start 184.8717 74.627) (end 184.8717 73.7753) (width 0.2) (layer "F.Cu") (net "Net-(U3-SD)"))
 (segment (start 186.7122 72.9008) (end 187.4129 73.6015) (width 0.2) (layer "F.Cu") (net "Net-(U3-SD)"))
 (segment (start 185.7462 72.9008) (end 186.7122 72.9008) (width 0.2) (layer "F.Cu") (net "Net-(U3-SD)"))
 (segment (start 187.4129 80.9471) (end 186.26 82.1) (width 0.2) (layer "F.Cu") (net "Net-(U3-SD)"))
 (segment (start 184.2137 75.285) (end 184.8717 74.627) (width 0.2) (layer "F.Cu") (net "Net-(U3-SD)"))
 (segment (start 176.77 43.6817) (end 188.1042 55.0159) (width 0.2) (layer "F.Cu") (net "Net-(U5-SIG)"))
 (segment (start 188.1042 81.8978) (end 186.7486 83.2534) (width 0.2) (layer "F.Cu") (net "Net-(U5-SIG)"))
 (segment (start 171.02 74.0863) (end 171.02 73.95) (width 0.2) (layer "F.Cu") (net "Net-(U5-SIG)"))
 (segment (start 184.2245 80.9483) (end 183.1682 80.9483) (width 0.2) (layer "F.Cu") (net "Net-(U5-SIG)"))
 (segment (start 182.2146 83.2517) (end 180.1854 83.2517) (width 0.2) (layer "F.Cu") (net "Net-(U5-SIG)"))
 (segment (start 186.7486 83.2534) (end 185.7133 83.2534) (width 0.2) (layer "F.Cu") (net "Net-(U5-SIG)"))
 (segment (start 184.8717 81.5955) (end 184.2245 80.9483) (width 0.2) (layer "F.Cu") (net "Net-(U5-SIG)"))
 (segment (start 180.1854 83.2517) (end 171.02 74.0863) (width 0.2) (layer "F.Cu") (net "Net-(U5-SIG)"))
 (segment (start 183.1682 80.9483) (end 182.45 81.6665) (width 0.2) (layer "F.Cu") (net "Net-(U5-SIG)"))
 (segment (start 185.7133 83.2534) (end 184.8717 82.4118) (width 0.2) (layer "F.Cu") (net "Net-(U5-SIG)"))
 (segment (start 188.1042 55.0159) (end 188.1042 81.8978) (width 0.2) (layer "F.Cu") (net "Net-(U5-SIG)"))
 (segment (start 182.45 83.0163) (end 182.2146 83.2517) (width 0.2) (layer "F.Cu") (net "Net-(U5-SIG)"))
 (segment (start 176.77 42.53) (end 176.77 43.6817) (width 0.2) (layer "F.Cu") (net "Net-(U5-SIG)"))
 (segment (start 184.8717 82.4118) (end 184.8717 81.5955) (width 0.2) (layer "F.Cu") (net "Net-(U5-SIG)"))
 (segment (start 182.45 81.6665) (end 182.45 83.0163) (width 0.2) (layer "F.Cu") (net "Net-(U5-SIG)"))
 (segment (start 182.7434 29.1703) (end 182.5779 29.3358) (width 0.2) (layer "F.Cu") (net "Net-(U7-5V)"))
 (segment (start 186.93 41.3783) (end 188.4672 39.8411) (width 0.2) (layer "F.Cu") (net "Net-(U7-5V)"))
 (segment (start 126.3859 29.3358) (end 123.4417 32.28) (width 0.2) (layer "F.Cu") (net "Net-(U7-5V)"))
 (segment (start 187.3314 28.9349) (end 182.9788 28.9349) (width 0.2) (layer "F.Cu") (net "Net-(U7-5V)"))
 (segment (start 182.7434 29.1703) (end 182.5779 29.3358) (width 0.2) (layer "F.Cu") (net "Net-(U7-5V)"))
 (segment (start 188.4672 39.8411) (end 188.4672 30.0707) (width 0.2) (layer "F.Cu") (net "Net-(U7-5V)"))
 (segment (start 121.94 32.28) (end 123.4417 32.28) (width 0.2) (layer "F.Cu") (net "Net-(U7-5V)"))
 (segment (start 182.5779 29.3358) (end 126.3859 29.3358) (width 0.2) (layer "F.Cu") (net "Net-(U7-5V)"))
 (segment (start 188.4672 30.0707) (end 187.3314 28.9349) (width 0.2) (layer "F.Cu") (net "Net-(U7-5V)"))
 (segment (start 182.9788 28.9349) (end 182.7434 29.1703) (width 0.2) (layer "F.Cu") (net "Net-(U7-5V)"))
 (segment (start 186.93 42.53) (end 186.93 41.3783) (width 0.2) (layer "F.Cu") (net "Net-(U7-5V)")))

